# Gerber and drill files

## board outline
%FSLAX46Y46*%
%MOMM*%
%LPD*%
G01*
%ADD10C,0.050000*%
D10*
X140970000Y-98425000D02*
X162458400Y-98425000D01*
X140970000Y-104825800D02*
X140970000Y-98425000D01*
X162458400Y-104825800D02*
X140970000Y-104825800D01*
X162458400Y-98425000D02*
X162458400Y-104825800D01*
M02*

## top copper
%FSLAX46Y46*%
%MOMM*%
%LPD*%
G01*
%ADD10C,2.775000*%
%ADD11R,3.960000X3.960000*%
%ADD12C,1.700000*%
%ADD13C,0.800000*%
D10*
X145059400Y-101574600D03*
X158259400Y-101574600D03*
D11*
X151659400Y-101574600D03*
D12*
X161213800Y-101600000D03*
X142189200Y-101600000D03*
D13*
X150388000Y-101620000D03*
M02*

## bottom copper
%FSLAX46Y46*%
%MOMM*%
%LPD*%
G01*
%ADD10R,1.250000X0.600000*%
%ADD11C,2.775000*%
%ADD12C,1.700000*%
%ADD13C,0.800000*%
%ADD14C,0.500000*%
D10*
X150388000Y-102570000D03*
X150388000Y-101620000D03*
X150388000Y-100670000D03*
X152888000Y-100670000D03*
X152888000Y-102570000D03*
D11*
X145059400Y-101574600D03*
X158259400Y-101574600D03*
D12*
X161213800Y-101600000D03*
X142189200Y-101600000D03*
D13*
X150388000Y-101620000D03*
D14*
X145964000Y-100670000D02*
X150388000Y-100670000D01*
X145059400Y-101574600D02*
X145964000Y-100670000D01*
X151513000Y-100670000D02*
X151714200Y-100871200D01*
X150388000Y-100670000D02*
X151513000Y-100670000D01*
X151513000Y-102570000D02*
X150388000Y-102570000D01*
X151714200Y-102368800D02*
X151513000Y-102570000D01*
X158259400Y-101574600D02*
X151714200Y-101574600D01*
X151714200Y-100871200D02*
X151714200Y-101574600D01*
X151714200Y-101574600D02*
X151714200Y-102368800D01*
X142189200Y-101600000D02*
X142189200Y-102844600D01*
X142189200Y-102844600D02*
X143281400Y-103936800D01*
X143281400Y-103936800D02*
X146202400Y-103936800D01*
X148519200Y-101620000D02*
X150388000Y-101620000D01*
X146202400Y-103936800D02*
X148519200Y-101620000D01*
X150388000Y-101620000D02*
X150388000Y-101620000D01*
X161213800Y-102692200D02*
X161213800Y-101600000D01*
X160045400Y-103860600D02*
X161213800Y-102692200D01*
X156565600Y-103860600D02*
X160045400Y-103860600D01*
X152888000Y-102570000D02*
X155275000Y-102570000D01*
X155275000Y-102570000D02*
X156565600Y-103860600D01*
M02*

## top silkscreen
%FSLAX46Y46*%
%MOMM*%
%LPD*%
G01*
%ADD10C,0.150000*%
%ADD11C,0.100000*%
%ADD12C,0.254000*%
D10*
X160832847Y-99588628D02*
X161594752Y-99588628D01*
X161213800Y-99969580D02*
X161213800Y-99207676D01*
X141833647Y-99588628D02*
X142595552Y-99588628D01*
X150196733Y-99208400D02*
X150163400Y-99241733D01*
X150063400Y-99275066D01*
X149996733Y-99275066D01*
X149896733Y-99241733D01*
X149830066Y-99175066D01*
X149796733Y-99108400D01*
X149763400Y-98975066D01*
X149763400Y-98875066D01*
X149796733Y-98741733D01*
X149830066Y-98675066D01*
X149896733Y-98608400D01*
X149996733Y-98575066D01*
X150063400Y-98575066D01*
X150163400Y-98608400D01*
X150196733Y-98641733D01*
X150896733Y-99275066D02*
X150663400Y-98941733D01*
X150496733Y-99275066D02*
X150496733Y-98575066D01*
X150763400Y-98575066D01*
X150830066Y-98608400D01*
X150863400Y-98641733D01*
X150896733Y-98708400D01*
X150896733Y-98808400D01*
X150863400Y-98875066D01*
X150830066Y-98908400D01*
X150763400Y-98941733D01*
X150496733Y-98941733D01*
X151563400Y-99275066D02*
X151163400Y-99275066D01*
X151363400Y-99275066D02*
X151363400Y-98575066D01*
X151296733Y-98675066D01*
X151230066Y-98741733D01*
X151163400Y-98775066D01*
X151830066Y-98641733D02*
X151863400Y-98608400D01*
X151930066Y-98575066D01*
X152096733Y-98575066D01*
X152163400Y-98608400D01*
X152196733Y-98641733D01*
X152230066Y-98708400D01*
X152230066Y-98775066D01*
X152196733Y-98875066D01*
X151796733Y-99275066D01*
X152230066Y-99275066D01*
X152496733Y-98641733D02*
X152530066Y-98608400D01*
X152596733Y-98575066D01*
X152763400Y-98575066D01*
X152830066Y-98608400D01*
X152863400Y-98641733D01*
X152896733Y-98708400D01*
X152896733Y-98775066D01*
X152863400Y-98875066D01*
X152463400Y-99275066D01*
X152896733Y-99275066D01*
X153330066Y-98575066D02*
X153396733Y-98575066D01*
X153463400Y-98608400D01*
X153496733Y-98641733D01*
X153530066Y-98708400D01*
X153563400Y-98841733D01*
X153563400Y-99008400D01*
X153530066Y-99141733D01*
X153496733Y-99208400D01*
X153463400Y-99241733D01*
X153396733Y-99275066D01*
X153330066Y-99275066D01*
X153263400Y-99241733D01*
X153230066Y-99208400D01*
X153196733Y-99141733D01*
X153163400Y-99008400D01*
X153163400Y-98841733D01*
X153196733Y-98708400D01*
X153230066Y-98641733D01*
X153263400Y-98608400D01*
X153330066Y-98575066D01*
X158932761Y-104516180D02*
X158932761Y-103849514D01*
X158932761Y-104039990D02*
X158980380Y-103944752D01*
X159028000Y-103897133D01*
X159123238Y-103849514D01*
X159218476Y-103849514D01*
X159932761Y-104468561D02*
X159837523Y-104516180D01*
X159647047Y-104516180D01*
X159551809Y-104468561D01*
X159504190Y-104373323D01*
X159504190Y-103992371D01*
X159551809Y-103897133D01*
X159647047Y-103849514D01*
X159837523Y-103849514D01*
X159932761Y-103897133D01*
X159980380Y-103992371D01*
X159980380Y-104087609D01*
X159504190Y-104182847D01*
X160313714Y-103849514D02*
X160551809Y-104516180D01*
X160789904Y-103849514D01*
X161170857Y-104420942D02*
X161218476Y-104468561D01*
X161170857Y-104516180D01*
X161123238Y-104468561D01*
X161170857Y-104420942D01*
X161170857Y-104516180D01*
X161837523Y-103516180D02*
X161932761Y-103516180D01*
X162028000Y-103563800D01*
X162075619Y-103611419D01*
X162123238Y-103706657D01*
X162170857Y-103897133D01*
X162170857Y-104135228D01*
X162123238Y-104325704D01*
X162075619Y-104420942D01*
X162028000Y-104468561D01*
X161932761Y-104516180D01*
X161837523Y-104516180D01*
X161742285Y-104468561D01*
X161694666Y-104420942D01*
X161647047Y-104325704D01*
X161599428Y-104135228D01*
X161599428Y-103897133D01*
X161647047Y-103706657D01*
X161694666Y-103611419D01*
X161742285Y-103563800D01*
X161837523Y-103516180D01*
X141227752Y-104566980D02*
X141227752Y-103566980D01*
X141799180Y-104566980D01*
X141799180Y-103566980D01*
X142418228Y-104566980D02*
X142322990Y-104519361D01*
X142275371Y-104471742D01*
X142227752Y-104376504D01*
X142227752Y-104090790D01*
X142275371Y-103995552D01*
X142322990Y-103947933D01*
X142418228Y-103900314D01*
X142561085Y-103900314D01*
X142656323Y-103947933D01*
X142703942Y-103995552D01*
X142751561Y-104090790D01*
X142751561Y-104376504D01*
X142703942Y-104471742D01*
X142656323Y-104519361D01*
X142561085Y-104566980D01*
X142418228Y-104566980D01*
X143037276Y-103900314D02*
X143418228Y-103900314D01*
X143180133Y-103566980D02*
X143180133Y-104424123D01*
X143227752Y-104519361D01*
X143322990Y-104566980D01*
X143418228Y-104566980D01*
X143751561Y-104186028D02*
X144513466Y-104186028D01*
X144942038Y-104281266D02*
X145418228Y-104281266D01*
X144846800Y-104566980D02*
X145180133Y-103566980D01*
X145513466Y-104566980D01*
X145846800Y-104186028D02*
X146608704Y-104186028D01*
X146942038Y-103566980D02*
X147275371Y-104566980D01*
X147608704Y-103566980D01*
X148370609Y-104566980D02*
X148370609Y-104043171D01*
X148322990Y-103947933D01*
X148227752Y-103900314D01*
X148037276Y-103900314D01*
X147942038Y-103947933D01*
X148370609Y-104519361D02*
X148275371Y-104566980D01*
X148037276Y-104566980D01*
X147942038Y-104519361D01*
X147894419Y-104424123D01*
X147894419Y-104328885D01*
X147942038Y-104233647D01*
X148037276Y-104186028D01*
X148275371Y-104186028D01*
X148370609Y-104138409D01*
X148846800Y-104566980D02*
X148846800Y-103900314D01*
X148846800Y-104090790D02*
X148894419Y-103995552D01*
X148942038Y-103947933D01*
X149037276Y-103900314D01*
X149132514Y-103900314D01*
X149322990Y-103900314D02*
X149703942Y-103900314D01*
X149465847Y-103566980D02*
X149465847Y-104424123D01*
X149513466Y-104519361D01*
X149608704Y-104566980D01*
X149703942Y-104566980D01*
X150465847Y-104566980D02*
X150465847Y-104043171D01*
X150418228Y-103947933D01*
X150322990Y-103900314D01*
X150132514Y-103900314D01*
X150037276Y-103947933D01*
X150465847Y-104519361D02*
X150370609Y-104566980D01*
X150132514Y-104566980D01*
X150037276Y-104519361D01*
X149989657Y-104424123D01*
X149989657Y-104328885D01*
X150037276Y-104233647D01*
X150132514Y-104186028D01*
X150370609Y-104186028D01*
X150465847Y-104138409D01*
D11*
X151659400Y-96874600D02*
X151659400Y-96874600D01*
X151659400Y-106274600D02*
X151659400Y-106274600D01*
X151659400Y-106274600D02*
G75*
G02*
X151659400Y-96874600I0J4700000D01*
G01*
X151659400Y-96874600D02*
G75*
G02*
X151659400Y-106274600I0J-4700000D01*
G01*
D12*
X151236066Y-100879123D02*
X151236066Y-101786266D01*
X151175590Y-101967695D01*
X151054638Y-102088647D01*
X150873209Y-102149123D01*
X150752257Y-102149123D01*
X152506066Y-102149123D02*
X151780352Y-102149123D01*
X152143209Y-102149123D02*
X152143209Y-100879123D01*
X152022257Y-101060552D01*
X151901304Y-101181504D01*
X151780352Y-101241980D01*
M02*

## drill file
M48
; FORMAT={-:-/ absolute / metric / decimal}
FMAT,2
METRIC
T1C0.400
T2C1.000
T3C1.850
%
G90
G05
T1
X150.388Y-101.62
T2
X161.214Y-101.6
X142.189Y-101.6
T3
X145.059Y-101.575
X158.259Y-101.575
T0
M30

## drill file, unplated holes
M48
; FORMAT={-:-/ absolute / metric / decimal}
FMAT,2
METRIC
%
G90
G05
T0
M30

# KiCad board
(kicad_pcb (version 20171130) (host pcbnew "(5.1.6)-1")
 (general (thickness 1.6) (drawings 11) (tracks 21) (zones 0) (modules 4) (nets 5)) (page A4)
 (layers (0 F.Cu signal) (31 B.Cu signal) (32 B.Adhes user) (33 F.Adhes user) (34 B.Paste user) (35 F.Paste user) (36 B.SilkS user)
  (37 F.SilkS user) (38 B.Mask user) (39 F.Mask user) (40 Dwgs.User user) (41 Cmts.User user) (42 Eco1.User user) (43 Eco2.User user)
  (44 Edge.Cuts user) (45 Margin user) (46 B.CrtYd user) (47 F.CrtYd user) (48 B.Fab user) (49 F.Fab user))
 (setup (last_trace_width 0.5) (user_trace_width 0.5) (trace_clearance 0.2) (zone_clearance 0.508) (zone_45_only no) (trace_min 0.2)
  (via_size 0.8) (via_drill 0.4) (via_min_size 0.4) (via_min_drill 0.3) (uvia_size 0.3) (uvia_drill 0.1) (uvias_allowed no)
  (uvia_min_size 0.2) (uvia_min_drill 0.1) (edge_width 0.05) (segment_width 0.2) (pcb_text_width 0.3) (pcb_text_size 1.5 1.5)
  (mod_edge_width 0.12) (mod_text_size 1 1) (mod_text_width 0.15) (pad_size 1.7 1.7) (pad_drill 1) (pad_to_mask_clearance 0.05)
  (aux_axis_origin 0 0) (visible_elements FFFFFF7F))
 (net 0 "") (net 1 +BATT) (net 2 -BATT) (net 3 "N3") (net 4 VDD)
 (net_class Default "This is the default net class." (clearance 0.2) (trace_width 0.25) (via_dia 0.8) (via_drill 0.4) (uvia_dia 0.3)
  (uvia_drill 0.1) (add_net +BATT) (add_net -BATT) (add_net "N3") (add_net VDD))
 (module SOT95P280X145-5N (layer B.Cu) (at 151.638 101.62)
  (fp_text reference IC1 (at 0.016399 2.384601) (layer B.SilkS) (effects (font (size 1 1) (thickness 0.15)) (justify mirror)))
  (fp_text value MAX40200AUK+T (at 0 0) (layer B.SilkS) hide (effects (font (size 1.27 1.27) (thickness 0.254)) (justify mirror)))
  (pad 1 smd rect (at -1.25 0.95 270) (size 0.6 1.25) (layers B.Cu B.Paste B.Mask) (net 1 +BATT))
  (pad 2 smd rect (at -1.25 0 270) (size 0.6 1.25) (layers B.Cu B.Paste B.Mask) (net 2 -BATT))
  (pad 3 smd rect (at -1.25 -0.95 270) (size 0.6 1.25) (layers B.Cu B.Paste B.Mask) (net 1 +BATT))
  (pad 4 smd rect (at 1.25 -0.95 270) (size 0.6 1.25) (layers B.Cu B.Paste B.Mask) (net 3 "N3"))
  (pad 5 smd rect (at 1.25 0.95 270) (size 0.6 1.25) (layers B.Cu B.Paste B.Mask) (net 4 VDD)))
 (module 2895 (layer F.Cu) (at 145.0594 101.5746)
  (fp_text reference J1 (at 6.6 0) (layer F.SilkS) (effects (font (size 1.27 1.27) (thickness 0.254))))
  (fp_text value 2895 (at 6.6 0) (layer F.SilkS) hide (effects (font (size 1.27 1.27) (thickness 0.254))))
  (fp_line (start 6.6 -4.7) (end 6.6 -4.7) (layer F.SilkS) (width 0.1))
  (fp_line (start 6.6 4.7) (end 6.6 4.7) (layer F.SilkS) (width 0.1))
  (fp_arc (start 6.6 0) (end 6.6 -4.7) (angle -180) (layer F.SilkS) (width 0.1))
  (fp_arc (start 6.6 0) (end 6.6 4.7) (angle -180) (layer F.SilkS) (width 0.1))
  (pad 1 thru_hole circle (at 0 0) (size 2.775 2.775) (drill 1.85) (layers *.Cu *.Mask) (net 1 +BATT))
  (pad 2 thru_hole circle (at 13.2 0) (size 2.775 2.775) (drill 1.85) (layers *.Cu *.Mask) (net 1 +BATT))
  (pad MP1 smd rect (at 6.6 0 90) (size 3.96 3.96) (layers F.Cu F.Paste F.Mask) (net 2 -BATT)))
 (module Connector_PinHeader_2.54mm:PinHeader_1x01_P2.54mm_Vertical (layer B.Cu) (at 161.2138 101.6)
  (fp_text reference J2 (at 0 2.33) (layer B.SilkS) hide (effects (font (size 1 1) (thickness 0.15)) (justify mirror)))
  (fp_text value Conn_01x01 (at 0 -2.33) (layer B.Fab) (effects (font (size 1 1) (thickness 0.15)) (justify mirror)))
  (pad 1 thru_hole circle (at 0 0) (size 1.7 1.7) (drill 1) (layers *.Cu *.Mask) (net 4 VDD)))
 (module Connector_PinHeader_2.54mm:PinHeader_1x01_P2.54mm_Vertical (layer B.Cu) (at 142.1892 101.6)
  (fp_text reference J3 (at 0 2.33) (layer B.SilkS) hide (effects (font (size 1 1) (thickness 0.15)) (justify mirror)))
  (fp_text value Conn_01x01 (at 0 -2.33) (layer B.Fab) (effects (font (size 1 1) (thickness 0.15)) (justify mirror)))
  (pad 1 thru_hole circle (at 0 0) (size 1.7 1.7) (drill 1) (layers *.Cu *.Mask) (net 2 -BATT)))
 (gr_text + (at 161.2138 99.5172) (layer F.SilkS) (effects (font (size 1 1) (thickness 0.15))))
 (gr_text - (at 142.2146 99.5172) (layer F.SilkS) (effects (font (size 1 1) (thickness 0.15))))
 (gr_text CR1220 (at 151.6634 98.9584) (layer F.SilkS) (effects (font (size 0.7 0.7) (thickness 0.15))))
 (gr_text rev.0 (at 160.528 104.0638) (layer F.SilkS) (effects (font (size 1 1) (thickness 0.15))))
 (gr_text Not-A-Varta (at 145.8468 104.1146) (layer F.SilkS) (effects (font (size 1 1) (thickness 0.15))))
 (gr_line (start 140.97 98.425) (end 162.4584 98.425) (layer Edge.Cuts) (width 0.05))
 (gr_line (start 140.97 104.8258) (end 140.97 98.425) (layer Edge.Cuts) (width 0.05))
 (gr_line (start 162.4584 104.8258) (end 140.97 104.8258) (layer Edge.Cuts) (width 0.05))
 (gr_line (start 162.4584 98.425) (end 162.4584 104.8258) (layer Edge.Cuts) (width 0.05))
 (segment (start 145.964 100.67) (end 150.388 100.67) (width 0.5) (layer B.Cu) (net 1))
 (segment (start 145.0594 101.5746) (end 145.964 100.67) (width 0.5) (layer B.Cu) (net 1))
 (segment (start 151.513 100.67) (end 151.7142 100.8712) (width 0.5) (layer B.Cu) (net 1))
 (segment (start 150.388 100.67) (end 151.513 100.67) (width 0.5) (layer B.Cu) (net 1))
 (segment (start 151.513 102.57) (end 150.388 102.57) (width 0.5) (layer B.Cu) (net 1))
 (segment (start 151.7142 102.3688) (end 151.513 102.57) (width 0.5) (layer B.Cu) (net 1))
 (segment (start 158.2594 101.5746) (end 151.7142 101.5746) (width 0.5) (layer B.Cu) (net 1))
 (segment (start 151.7142 100.8712) (end 151.7142 101.5746) (width 0.5) (layer B.Cu) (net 1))
 (segment (start 151.7142 101.5746) (end 151.7142 102.3688) (width 0.5) (layer B.Cu) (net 1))
 (segment (start 142.1892 101.6) (end 142.1892 102.8446) (width 0.5) (layer B.Cu) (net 2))
 (segment (start 142.1892 102.8446) (end 143.2814 103.9368) (width 0.5) (layer B.Cu) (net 2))
 (segment (start 143.2814 103.9368) (end 146.2024 103.9368) (width 0.5) (layer B.Cu) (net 2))
 (segment (start 148.5192 101.62) (end 150.388 101.62) (width 0.5) (layer B.Cu) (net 2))
 (segment (start 146.2024 103.9368) (end 148.5192 101.62) (width 0.5) (layer B.Cu) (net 2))
 (segment (start 150.388 101.62) (end 150.388 101.62) (width 0.5) (layer B.Cu) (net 2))
 (via (at 150.388 101.62) (size 0.8) (drill 0.4) (layers F.Cu B.Cu) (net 2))
 (segment (start 161.2138 102.6922) (end 161.2138 101.6) (width 0.5) (layer B.Cu) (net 4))
 (segment (start 160.0454 103.8606) (end 161.2138 102.6922) (width 0.5) (layer B.Cu) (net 4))
 (segment (start 156.5656 103.8606) (end 160.0454 103.8606) (width 0.5) (layer B.Cu) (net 4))
 (segment (start 152.888 102.57) (end 155.275 102.57) (width 0.5) (layer B.Cu) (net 4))
 (segment (start 155.275 102.57) (end 156.5656 103.8606) (width 0.5) (layer B.Cu) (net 4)))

